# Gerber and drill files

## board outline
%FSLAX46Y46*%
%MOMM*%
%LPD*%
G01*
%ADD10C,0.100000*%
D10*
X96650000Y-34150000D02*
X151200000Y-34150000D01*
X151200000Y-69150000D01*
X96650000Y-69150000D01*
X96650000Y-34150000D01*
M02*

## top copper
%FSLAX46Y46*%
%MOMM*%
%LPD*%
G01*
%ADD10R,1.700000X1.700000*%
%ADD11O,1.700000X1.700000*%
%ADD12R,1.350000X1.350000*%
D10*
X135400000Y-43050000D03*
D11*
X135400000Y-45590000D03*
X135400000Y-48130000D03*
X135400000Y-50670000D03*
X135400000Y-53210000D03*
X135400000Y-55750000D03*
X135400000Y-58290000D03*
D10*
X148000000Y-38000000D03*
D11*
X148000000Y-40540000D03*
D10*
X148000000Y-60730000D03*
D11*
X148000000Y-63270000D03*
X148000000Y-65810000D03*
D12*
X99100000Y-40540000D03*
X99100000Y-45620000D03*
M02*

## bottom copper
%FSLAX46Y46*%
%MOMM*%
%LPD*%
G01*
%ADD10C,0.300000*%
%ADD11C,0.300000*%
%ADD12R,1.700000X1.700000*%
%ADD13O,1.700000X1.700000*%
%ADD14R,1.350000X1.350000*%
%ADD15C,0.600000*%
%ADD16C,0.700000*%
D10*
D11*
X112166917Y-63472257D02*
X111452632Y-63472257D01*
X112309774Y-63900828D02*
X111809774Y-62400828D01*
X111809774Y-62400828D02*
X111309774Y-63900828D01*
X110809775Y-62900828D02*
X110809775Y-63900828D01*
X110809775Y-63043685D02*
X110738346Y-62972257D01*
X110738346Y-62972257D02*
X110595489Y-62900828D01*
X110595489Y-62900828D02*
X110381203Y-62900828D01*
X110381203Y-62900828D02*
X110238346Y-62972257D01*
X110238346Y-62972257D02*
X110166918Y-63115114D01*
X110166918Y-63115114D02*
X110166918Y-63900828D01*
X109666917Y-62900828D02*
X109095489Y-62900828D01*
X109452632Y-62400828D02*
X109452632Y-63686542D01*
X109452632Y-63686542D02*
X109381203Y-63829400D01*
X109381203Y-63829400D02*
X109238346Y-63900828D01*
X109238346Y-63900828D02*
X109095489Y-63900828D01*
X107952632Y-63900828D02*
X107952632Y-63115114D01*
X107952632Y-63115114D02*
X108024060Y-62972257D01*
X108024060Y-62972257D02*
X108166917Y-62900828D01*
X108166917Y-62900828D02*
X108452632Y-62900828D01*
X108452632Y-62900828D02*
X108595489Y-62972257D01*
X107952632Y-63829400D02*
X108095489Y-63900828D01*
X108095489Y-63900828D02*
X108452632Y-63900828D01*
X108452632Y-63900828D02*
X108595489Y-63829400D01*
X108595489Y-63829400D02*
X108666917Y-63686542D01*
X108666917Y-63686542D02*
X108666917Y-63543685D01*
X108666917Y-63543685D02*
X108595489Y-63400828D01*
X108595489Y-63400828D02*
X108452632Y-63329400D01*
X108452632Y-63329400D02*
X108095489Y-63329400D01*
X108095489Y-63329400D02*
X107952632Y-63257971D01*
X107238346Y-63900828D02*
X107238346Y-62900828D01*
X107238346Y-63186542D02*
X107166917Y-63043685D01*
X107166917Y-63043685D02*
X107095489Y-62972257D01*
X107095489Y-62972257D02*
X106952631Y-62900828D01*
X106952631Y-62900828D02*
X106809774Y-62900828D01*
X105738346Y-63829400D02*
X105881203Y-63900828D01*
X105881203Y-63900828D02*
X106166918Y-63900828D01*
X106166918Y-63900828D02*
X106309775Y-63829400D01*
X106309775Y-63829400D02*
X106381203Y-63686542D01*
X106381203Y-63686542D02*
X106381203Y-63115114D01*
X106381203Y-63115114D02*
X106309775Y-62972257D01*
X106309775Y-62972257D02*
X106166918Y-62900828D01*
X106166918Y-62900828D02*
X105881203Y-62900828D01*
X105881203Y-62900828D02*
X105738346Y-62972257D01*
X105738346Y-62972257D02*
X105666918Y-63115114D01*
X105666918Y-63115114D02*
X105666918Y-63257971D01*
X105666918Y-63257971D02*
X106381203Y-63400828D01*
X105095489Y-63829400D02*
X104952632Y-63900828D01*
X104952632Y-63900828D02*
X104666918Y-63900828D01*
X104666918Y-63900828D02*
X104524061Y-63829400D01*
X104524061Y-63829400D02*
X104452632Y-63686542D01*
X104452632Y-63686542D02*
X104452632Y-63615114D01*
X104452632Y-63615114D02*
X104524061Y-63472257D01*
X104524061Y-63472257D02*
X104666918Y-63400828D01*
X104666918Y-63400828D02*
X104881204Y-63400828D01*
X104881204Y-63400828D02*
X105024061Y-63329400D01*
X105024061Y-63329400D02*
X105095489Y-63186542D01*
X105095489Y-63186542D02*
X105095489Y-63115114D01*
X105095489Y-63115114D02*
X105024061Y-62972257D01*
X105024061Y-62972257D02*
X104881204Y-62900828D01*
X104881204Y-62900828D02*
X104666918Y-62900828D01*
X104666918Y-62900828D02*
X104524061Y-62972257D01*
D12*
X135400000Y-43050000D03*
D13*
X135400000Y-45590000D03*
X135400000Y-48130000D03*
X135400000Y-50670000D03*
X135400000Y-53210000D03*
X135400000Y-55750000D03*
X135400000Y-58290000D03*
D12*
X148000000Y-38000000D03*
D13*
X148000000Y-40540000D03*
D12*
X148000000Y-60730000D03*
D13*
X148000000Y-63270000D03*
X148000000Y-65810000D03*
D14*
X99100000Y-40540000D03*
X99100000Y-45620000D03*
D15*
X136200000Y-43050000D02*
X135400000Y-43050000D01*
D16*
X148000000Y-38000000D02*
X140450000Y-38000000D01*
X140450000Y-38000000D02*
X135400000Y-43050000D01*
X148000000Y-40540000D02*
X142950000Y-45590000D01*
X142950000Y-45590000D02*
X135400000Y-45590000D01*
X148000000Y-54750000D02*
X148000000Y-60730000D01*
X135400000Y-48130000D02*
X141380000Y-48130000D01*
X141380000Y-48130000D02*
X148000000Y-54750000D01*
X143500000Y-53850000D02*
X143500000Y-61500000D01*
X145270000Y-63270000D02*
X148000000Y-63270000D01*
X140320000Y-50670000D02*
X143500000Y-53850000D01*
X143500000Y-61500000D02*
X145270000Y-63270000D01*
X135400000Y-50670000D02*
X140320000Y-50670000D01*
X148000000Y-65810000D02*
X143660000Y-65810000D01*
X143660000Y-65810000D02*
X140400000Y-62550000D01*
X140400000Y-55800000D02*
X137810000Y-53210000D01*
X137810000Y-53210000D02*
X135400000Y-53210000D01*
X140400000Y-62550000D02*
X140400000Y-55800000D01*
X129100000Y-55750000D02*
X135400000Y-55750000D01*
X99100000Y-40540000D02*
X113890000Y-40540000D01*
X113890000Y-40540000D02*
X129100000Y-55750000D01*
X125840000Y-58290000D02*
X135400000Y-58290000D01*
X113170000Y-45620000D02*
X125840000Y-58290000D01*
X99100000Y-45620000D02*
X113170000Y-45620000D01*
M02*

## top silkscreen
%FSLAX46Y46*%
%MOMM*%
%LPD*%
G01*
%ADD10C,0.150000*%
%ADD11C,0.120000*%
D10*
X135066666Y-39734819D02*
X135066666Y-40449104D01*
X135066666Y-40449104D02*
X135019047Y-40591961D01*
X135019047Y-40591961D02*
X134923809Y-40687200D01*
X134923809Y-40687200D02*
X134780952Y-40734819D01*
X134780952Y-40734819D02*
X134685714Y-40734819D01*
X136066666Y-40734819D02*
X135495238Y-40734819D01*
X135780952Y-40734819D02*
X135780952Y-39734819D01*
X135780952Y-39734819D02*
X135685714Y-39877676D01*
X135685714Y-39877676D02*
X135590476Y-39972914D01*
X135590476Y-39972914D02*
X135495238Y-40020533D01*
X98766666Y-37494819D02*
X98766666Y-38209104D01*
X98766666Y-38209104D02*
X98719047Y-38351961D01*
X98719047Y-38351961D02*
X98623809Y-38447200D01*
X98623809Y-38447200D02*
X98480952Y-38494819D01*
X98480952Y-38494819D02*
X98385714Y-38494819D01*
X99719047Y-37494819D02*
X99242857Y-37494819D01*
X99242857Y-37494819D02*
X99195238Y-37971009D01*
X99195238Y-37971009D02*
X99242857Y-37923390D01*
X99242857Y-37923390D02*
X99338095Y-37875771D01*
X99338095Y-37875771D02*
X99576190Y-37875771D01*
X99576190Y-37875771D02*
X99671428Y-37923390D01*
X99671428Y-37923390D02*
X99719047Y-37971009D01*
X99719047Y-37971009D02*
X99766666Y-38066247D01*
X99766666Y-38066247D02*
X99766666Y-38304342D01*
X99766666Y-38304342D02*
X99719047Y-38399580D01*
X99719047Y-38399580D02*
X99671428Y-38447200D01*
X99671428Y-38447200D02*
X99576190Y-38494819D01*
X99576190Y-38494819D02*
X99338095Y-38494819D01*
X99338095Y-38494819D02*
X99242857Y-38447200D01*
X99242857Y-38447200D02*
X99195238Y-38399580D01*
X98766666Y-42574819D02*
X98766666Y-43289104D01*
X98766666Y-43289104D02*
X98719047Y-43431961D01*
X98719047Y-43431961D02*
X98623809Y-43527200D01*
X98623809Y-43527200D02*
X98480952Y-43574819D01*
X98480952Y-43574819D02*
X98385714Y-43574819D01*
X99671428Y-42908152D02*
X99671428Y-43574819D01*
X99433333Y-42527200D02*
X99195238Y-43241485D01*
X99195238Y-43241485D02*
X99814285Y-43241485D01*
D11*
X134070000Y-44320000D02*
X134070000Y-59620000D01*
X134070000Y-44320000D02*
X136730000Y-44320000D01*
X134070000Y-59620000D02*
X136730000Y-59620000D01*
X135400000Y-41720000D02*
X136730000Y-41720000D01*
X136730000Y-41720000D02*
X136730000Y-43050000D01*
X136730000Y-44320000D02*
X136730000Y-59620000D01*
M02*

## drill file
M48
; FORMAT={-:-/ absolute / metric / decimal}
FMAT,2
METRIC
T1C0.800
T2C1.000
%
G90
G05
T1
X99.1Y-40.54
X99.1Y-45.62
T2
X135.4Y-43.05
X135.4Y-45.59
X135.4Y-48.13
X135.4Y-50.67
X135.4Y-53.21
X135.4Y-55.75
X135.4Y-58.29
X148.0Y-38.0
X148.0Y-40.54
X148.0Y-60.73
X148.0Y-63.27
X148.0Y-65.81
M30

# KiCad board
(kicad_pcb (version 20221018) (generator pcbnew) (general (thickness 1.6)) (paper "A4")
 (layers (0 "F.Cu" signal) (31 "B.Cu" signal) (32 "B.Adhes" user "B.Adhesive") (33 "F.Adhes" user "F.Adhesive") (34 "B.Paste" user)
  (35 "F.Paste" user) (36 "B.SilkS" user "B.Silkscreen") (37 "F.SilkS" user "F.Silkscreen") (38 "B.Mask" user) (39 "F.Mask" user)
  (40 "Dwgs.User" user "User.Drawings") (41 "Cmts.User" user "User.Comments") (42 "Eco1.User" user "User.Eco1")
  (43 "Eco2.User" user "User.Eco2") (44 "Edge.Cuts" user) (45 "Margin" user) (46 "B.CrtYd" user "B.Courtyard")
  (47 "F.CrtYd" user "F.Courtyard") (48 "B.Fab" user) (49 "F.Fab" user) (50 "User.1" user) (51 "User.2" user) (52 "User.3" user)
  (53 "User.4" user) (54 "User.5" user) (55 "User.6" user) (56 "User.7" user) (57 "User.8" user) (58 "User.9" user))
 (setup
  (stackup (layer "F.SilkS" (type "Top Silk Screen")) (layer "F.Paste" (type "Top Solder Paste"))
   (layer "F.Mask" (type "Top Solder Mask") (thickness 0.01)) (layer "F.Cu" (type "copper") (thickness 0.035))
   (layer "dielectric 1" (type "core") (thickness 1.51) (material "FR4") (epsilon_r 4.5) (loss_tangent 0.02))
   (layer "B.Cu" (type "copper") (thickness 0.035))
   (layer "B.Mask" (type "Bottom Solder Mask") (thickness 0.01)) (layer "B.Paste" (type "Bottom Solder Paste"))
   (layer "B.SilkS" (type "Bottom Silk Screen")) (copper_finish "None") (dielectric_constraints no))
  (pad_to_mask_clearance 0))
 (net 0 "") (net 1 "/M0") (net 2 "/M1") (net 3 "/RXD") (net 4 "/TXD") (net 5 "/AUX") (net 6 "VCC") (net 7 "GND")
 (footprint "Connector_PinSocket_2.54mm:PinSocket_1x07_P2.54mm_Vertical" (layer "F.Cu") (at 135.4 43.05)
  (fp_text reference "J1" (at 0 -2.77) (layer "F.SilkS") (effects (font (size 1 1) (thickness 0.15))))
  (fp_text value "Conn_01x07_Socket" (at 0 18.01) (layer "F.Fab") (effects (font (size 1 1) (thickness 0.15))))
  (fp_line (start -1.33 1.27) (end -1.33 16.57) (stroke (width 0.12) (type solid)) (layer "F.SilkS"))
  (fp_line (start -1.33 1.27) (end 1.33 1.27) (stroke (width 0.12) (type solid)) (layer "F.SilkS"))
  (fp_line (start -1.33 16.57) (end 1.33 16.57) (stroke (width 0.12) (type solid)) (layer "F.SilkS"))
  (fp_line (start 0 -1.33) (end 1.33 -1.33) (stroke (width 0.12) (type solid)) (layer "F.SilkS"))
  (fp_line (start 1.33 -1.33) (end 1.33 0) (stroke (width 0.12) (type solid)) (layer "F.SilkS"))
  (fp_line (start 1.33 1.27) (end 1.33 16.57) (stroke (width 0.12) (type solid)) (layer "F.SilkS"))
  (pad "1" thru_hole rect (at 0 0) (size 1.7 1.7) (drill 1) (layers "*.Cu" "*.Mask") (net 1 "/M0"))
  (pad "2" thru_hole oval (at 0 2.54) (size 1.7 1.7) (drill 1) (layers "*.Cu" "*.Mask") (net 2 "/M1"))
  (pad "3" thru_hole oval (at 0 5.08) (size 1.7 1.7) (drill 1) (layers "*.Cu" "*.Mask") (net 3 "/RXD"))
  (pad "4" thru_hole oval (at 0 7.62) (size 1.7 1.7) (drill 1) (layers "*.Cu" "*.Mask") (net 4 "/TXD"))
  (pad "5" thru_hole oval (at 0 10.16) (size 1.7 1.7) (drill 1) (layers "*.Cu" "*.Mask") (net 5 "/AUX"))
  (pad "6" thru_hole oval (at 0 12.7) (size 1.7 1.7) (drill 1) (layers "*.Cu" "*.Mask") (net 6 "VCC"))
  (pad "7" thru_hole oval (at 0 15.24) (size 1.7 1.7) (drill 1) (layers "*.Cu" "*.Mask") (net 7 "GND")))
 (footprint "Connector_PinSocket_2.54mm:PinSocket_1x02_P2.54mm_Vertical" (layer "B.Cu") (at 148 38 180)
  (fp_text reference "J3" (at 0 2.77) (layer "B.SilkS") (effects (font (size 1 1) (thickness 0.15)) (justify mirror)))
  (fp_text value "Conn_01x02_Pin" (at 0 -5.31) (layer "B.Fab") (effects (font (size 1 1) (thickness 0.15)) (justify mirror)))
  (pad "1" thru_hole rect (at 0 0 180) (size 1.7 1.7) (drill 1) (layers "*.Cu" "*.Mask") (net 1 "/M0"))
  (pad "2" thru_hole oval (at 0 -2.54 180) (size 1.7 1.7) (drill 1) (layers "*.Cu" "*.Mask") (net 2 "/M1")))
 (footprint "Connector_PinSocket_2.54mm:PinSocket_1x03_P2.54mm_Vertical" (layer "B.Cu") (at 148 60.73 180)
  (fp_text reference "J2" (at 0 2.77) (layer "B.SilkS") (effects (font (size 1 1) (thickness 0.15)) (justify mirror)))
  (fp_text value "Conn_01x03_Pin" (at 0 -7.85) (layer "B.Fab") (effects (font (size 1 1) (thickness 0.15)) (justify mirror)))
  (pad "1" thru_hole rect (at 0 0 180) (size 1.7 1.7) (drill 1) (layers "*.Cu" "*.Mask") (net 3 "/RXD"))
  (pad "2" thru_hole oval (at 0 -2.54 180) (size 1.7 1.7) (drill 1) (layers "*.Cu" "*.Mask") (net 4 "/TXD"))
  (pad "3" thru_hole oval (at 0 -5.08 180) (size 1.7 1.7) (drill 1) (layers "*.Cu" "*.Mask") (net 5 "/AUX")))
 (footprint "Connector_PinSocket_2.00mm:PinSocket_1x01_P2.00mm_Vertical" (layer "B.Cu") (at 99.1 40.54 180)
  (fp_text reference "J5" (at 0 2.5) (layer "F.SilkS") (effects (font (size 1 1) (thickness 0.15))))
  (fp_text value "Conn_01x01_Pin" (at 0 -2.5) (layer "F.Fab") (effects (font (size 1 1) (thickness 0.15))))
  (pad "1" thru_hole rect (at 0 0 180) (size 1.35 1.35) (drill 0.8) (layers "*.Cu" "*.Mask") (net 6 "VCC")))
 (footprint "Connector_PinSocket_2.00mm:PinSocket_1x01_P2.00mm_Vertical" (layer "B.Cu") (at 99.1 45.62 180)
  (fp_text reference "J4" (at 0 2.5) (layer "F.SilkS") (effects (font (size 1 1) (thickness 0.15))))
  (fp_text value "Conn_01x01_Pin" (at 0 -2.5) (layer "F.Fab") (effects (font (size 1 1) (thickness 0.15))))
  (pad "1" thru_hole rect (at 0 0 180) (size 1.35 1.35) (drill 0.8) (layers "*.Cu" "*.Mask") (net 7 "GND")))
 (gr_rect (start 96.65 34.15) (end 151.2 69.15) (stroke (width 0.1) (type default)) (fill none) (layer "Edge.Cuts"))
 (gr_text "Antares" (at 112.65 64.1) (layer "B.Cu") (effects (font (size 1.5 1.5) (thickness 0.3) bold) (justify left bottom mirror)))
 (segment (start 136.2 43.05) (end 135.4 43.05) (width 0.6) (layer "B.Cu") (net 1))
 (segment (start 148 38) (end 140.45 38) (width 0.7) (layer "B.Cu") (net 1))
 (segment (start 140.45 38) (end 135.4 43.05) (width 0.7) (layer "B.Cu") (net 1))
 (segment (start 148 40.54) (end 142.95 45.59) (width 0.7) (layer "B.Cu") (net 2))
 (segment (start 142.95 45.59) (end 135.4 45.59) (width 0.7) (layer "B.Cu") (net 2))
 (segment (start 148 54.75) (end 148 60.73) (width 0.7) (layer "B.Cu") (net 3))
 (segment (start 135.4 48.13) (end 141.38 48.13) (width 0.7) (layer "B.Cu") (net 3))
 (segment (start 141.38 48.13) (end 148 54.75) (width 0.7) (layer "B.Cu") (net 3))
 (segment (start 143.5 53.85) (end 143.5 61.5) (width 0.7) (layer "B.Cu") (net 4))
 (segment (start 145.27 63.27) (end 148 63.27) (width 0.7) (layer "B.Cu") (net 4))
 (segment (start 140.32 50.67) (end 143.5 53.85) (width 0.7) (layer "B.Cu") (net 4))
 (segment (start 143.5 61.5) (end 145.27 63.27) (width 0.7) (layer "B.Cu") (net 4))
 (segment (start 135.4 50.67) (end 140.32 50.67) (width 0.7) (layer "B.Cu") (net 4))
 (segment (start 148 65.81) (end 143.66 65.81) (width 0.7) (layer "B.Cu") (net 5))
 (segment (start 143.66 65.81) (end 140.4 62.55) (width 0.7) (layer "B.Cu") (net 5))
 (segment (start 140.4 55.8) (end 137.81 53.21) (width 0.7) (layer "B.Cu") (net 5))
 (segment (start 137.81 53.21) (end 135.4 53.21) (width 0.7) (layer "B.Cu") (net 5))
 (segment (start 140.4 62.55) (end 140.4 55.8) (width 0.7) (layer "B.Cu") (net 5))
 (segment (start 129.1 55.75) (end 135.4 55.75) (width 0.7) (layer "B.Cu") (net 6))
 (segment (start 99.1 40.54) (end 113.89 40.54) (width 0.7) (layer "B.Cu") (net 6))
 (segment (start 113.89 40.54) (end 129.1 55.75) (width 0.7) (layer "B.Cu") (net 6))
 (segment (start 125.84 58.29) (end 135.4 58.29) (width 0.7) (layer "B.Cu") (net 7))
 (segment (start 113.17 45.62) (end 125.84 58.29) (width 0.7) (layer "B.Cu") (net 7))
 (segment (start 99.1 45.62) (end 113.17 45.62) (width 0.7) (layer "B.Cu") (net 7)))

